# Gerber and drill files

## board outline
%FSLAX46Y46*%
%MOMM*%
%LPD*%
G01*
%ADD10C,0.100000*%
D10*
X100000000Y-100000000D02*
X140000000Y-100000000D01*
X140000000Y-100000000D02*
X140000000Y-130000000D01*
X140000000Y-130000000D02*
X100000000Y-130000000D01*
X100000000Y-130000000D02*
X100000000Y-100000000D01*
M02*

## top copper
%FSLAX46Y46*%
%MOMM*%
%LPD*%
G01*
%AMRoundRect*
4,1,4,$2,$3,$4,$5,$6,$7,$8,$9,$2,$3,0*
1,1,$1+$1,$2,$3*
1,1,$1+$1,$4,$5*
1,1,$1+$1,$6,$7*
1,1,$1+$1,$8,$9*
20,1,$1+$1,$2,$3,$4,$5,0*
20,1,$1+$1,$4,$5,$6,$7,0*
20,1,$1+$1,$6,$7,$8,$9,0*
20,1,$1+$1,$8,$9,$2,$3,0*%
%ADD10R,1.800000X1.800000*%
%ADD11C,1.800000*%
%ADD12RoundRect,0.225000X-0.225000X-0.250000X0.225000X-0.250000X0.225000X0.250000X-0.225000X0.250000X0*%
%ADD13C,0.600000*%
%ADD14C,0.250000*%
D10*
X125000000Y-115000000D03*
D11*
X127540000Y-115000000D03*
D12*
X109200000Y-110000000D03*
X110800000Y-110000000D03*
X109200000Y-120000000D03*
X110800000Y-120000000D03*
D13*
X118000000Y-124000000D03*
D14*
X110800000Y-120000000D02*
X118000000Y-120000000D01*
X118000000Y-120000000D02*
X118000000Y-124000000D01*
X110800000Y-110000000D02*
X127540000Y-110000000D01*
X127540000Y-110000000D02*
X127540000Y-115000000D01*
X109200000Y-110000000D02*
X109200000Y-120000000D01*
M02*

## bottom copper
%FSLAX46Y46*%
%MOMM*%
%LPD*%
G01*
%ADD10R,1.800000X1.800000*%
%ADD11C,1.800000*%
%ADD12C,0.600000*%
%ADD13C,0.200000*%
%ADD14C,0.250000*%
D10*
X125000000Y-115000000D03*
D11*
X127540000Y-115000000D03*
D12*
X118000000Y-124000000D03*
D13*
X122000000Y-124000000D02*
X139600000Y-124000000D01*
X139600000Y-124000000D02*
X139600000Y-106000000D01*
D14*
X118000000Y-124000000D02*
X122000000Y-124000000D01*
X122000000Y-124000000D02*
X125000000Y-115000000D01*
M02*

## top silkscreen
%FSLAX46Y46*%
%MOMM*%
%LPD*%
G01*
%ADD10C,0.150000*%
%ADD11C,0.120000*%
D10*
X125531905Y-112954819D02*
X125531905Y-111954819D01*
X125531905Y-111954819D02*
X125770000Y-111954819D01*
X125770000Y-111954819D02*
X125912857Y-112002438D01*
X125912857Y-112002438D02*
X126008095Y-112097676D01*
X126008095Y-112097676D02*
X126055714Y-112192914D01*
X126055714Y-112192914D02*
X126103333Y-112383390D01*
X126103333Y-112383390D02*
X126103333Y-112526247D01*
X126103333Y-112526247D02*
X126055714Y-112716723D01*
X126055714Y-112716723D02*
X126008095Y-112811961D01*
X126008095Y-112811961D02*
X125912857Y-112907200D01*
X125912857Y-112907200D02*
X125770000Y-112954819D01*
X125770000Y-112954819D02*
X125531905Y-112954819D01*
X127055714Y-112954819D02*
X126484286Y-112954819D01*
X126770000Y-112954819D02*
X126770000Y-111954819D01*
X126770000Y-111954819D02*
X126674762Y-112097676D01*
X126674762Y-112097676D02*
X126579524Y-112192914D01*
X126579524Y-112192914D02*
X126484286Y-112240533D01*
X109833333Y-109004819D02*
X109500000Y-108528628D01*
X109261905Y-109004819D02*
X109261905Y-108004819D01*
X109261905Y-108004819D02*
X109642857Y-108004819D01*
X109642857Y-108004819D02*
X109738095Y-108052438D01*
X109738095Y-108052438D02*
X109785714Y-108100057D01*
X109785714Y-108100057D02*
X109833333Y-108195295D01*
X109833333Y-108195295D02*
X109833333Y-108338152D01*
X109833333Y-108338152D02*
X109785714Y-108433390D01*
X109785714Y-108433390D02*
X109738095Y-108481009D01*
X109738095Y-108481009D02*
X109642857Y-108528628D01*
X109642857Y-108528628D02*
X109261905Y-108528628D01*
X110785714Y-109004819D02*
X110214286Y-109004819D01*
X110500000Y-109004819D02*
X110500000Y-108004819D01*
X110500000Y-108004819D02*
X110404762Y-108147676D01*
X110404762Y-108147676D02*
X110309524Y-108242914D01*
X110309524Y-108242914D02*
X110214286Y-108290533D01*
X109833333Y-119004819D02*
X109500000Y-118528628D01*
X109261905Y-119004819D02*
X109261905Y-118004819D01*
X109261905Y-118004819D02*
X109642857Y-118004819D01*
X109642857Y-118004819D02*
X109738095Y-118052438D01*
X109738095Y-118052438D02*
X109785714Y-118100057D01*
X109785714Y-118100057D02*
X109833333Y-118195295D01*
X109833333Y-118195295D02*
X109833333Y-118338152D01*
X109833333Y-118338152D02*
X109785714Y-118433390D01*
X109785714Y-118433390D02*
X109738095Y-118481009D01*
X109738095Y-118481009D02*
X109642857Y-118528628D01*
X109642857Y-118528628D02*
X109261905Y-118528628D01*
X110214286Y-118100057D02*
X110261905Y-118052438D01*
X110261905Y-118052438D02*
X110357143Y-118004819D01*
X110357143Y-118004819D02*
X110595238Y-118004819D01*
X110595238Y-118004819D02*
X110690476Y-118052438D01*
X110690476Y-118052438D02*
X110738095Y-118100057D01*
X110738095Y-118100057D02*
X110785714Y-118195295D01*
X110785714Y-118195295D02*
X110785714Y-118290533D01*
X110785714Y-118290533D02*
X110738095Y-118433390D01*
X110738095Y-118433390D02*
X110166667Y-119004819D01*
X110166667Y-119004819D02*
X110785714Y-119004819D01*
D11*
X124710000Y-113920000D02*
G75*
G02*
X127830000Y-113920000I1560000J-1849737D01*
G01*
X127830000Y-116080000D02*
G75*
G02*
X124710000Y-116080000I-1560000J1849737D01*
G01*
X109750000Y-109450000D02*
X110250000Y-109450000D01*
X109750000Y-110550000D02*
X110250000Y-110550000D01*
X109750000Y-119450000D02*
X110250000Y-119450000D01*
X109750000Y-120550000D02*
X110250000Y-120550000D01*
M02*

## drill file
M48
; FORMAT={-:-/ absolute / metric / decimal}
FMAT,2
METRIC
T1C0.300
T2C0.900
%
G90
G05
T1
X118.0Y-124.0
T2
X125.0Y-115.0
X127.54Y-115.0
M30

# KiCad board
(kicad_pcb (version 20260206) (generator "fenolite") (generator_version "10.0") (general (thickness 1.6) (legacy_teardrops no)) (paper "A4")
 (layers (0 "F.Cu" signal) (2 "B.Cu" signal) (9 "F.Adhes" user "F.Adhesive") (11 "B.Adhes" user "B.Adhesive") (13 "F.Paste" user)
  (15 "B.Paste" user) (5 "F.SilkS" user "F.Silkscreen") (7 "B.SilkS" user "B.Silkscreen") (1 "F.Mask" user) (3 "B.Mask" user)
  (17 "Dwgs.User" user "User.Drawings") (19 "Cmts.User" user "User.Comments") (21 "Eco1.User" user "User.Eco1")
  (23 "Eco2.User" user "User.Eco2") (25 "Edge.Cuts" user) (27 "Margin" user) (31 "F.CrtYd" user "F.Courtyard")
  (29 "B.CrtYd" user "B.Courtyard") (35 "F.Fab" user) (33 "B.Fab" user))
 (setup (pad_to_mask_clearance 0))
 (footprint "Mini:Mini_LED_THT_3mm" (layer "F.Cu") (at 125 115)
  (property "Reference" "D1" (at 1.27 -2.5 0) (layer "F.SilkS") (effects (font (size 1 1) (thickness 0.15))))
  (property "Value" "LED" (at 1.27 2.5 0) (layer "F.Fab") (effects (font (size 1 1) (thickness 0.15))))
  (fp_arc (start -0.29 -1.08) (mid 1.27 -1.65) (end 2.83 -1.08) (stroke (width 0.12) (type solid)) (layer "F.SilkS"))
  (fp_arc (start 2.83 1.08) (mid 1.27 1.65) (end -0.29 1.08) (stroke (width 0.12) (type solid)) (layer "F.SilkS"))
  (pad "1" thru_hole rect (at 0 0) (size 1.8 1.8) (drill 0.9) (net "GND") (layers "*.Cu" "*.Mask") (remove_unused_layers no))
  (pad "2" thru_hole circle (at 2.54 0) (size 1.8 1.8) (drill 0.9) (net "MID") (layers "*.Cu" "*.Mask") (remove_unused_layers no)))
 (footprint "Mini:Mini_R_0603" (layer "F.Cu") (at 110 110)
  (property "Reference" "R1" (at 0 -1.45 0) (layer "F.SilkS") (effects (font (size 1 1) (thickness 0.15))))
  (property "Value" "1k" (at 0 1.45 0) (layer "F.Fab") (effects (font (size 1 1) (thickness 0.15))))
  (fp_line (start -0.25 -0.55) (end 0.25 -0.55) (stroke (width 0.12) (type solid)) (layer "F.SilkS"))
  (fp_line (start -0.25 0.55) (end 0.25 0.55) (stroke (width 0.12) (type solid)) (layer "F.SilkS"))
  (pad "1" smd roundrect (at -0.8 0) (size 0.9 0.95) (layers "F.Cu" "F.Mask" "F.Paste") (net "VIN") (roundrect_rratio 0.25))
  (pad "2" smd roundrect (at 0.8 0) (size 0.9 0.95) (layers "F.Cu" "F.Mask" "F.Paste") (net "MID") (roundrect_rratio 0.25)))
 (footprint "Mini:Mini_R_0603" (layer "F.Cu") (at 110 120)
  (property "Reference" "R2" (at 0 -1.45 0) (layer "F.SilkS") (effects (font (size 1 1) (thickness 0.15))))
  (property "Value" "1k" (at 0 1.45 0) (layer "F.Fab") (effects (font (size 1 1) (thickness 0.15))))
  (fp_line (start -0.25 -0.55) (end 0.25 -0.55) (stroke (width 0.12) (type solid)) (layer "F.SilkS"))
  (fp_line (start -0.25 0.55) (end 0.25 0.55) (stroke (width 0.12) (type solid)) (layer "F.SilkS"))
  (pad "1" smd roundrect (at -0.8 0) (size 0.9 0.95) (layers "F.Cu" "F.Mask" "F.Paste") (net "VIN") (roundrect_rratio 0.25))
  (pad "2" smd roundrect (at 0.8 0) (size 0.9 0.95) (layers "F.Cu" "F.Mask" "F.Paste") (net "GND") (roundrect_rratio 0.25)))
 (gr_line (start 100 100) (end 140 100) (stroke (width 0.1) (type solid)) (layer "Edge.Cuts"))
 (gr_line (start 140 100) (end 140 130) (stroke (width 0.1) (type solid)) (layer "Edge.Cuts"))
 (gr_line (start 140 130) (end 100 130) (stroke (width 0.1) (type solid)) (layer "Edge.Cuts"))
 (gr_line (start 100 130) (end 100 100) (stroke (width 0.1) (type solid)) (layer "Edge.Cuts"))
 (segment (start 122 124) (end 139.6 124) (width 0.2) (layer "B.Cu") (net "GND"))
 (segment (start 139.6 124) (end 139.6 106) (width 0.2) (layer "B.Cu") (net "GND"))
 (segment (start 110.8 120) (end 118 120) (width 0.25) (layer "F.Cu") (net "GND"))
 (segment (start 118 120) (end 118 124) (width 0.25) (layer "F.Cu") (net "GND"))
 (segment (start 118 124) (end 122 124) (width 0.25) (layer "B.Cu") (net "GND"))
 (segment (start 122 124) (end 125 115) (width 0.25) (layer "B.Cu") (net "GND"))
 (segment (start 110.8 110) (end 127.54 110) (width 0.25) (layer "F.Cu") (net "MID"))
 (segment (start 127.54 110) (end 127.54 115) (width 0.25) (layer "F.Cu") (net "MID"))
 (segment (start 109.2 110) (end 109.2 120) (width 0.25) (layer "F.Cu") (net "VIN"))
 (via (at 118 124) (size 0.6) (drill 0.3) (layers "F.Cu" "B.Cu") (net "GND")))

